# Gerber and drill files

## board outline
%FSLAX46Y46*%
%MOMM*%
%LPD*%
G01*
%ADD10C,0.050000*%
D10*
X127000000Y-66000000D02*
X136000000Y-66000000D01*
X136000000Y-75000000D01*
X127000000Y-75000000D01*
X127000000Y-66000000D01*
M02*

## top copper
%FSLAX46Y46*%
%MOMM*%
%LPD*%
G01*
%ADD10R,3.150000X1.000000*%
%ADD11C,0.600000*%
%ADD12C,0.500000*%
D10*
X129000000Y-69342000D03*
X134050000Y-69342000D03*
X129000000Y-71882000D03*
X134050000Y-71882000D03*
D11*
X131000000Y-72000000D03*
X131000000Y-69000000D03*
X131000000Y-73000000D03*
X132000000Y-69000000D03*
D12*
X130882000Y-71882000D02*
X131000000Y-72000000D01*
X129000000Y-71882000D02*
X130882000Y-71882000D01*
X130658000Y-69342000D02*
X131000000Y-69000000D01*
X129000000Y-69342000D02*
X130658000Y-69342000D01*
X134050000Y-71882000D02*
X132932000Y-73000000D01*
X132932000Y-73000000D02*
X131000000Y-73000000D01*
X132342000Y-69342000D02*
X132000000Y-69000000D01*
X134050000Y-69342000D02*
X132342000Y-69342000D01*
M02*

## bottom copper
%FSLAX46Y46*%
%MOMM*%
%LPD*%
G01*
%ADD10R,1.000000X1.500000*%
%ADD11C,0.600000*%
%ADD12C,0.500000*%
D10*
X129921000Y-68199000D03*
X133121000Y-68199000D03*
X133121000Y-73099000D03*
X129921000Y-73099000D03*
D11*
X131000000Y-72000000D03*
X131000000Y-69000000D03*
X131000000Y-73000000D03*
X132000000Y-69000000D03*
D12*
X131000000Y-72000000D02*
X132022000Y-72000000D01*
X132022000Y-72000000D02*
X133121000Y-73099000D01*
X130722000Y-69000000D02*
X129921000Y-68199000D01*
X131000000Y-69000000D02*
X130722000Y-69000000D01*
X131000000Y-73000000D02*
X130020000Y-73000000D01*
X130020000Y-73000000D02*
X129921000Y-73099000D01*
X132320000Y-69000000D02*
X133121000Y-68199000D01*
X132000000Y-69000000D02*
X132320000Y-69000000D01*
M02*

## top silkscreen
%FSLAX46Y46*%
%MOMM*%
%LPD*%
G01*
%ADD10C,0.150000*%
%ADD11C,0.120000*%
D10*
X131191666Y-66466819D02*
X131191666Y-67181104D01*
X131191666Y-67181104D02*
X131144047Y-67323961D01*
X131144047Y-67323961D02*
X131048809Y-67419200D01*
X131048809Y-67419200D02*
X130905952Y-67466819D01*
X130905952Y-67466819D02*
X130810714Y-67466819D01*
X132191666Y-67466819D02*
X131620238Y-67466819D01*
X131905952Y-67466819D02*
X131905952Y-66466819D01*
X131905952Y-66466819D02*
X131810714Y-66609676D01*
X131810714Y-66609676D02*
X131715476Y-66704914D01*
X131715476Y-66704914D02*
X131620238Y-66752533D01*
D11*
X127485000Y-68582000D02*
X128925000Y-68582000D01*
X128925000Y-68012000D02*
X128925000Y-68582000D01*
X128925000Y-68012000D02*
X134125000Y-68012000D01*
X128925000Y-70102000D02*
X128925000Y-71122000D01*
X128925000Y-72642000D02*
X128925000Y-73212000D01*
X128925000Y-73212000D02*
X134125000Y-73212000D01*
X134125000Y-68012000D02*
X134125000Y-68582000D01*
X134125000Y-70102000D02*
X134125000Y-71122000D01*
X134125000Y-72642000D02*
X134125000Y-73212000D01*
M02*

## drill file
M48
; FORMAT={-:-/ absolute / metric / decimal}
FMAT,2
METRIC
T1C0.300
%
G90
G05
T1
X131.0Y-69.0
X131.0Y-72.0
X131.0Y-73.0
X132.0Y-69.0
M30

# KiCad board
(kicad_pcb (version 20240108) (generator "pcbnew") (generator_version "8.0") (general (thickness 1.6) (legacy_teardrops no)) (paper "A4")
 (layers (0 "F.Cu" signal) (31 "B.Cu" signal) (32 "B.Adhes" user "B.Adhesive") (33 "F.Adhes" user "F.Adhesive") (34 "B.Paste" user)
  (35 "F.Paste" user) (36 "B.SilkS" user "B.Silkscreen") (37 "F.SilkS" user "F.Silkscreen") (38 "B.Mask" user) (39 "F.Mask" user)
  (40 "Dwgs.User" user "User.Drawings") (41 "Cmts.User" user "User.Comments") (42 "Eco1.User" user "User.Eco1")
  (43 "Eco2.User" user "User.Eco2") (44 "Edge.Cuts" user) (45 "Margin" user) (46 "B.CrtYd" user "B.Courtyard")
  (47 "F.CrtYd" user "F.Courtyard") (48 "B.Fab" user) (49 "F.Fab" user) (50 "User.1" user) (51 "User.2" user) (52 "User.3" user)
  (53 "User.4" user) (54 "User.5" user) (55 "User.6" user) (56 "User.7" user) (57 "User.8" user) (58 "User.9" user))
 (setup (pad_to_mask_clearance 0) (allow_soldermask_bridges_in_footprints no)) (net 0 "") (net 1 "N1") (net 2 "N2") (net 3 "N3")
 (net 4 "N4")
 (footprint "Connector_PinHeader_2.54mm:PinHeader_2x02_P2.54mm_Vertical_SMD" (layer "F.Cu") (at 131.525 70.612)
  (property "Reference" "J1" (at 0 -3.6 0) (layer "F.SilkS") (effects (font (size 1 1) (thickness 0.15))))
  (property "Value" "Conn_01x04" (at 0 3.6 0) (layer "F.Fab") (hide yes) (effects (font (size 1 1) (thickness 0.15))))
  (fp_line (start -4.04 -2.03) (end -2.6 -2.03) (stroke (width 0.12) (type solid)) (layer "F.SilkS"))
  (fp_line (start -2.6 -2.6) (end -2.6 -2.03) (stroke (width 0.12) (type solid)) (layer "F.SilkS"))
  (fp_line (start -2.6 -2.6) (end 2.6 -2.6) (stroke (width 0.12) (type solid)) (layer "F.SilkS"))
  (fp_line (start -2.6 -0.51) (end -2.6 0.51) (stroke (width 0.12) (type solid)) (layer "F.SilkS"))
  (fp_line (start -2.6 2.03) (end -2.6 2.6) (stroke (width 0.12) (type solid)) (layer "F.SilkS"))
  (fp_line (start -2.6 2.6) (end 2.6 2.6) (stroke (width 0.12) (type solid)) (layer "F.SilkS"))
  (fp_line (start 2.6 -2.6) (end 2.6 -2.03) (stroke (width 0.12) (type solid)) (layer "F.SilkS"))
  (fp_line (start 2.6 -0.51) (end 2.6 0.51) (stroke (width 0.12) (type solid)) (layer "F.SilkS"))
  (fp_line (start 2.6 2.03) (end 2.6 2.6) (stroke (width 0.12) (type solid)) (layer "F.SilkS"))
  (pad "1" smd rect (at -2.525 -1.27) (size 3.15 1) (layers "F.Cu" "F.Paste" "F.Mask") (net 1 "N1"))
  (pad "2" smd rect (at 2.525 -1.27) (size 3.15 1) (layers "F.Cu" "F.Paste" "F.Mask") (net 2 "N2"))
  (pad "3" smd rect (at -2.525 1.27) (size 3.15 1) (layers "F.Cu" "F.Paste" "F.Mask") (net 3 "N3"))
  (pad "4" smd rect (at 2.525 1.27) (size 3.15 1) (layers "F.Cu" "F.Paste" "F.Mask") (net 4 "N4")))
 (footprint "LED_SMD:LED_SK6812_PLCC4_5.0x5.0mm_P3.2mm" (layer "B.Cu") (at 131.521 70.649 90)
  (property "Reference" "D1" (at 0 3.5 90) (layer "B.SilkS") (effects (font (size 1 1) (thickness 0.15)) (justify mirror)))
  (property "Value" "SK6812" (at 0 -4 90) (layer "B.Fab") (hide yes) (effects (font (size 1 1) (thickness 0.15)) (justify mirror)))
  (pad "1" smd rect (at 2.45 -1.6 90) (size 1.5 1) (layers "B.Cu" "B.Paste" "B.Mask") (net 1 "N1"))
  (pad "2" smd rect (at 2.45 1.6 90) (size 1.5 1) (layers "B.Cu" "B.Paste" "B.Mask") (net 2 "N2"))
  (pad "3" smd rect (at -2.45 1.6 90) (size 1.5 1) (layers "B.Cu" "B.Paste" "B.Mask") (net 3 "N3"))
  (pad "4" smd rect (at -2.45 -1.6 90) (size 1.5 1) (layers "B.Cu" "B.Paste" "B.Mask") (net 4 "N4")))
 (gr_rect (start 127 66) (end 136 75) (stroke (width 0.05) (type default)) (fill none) (layer "Edge.Cuts"))
 (segment (start 130.882 71.882) (end 131 72) (width 0.5) (layer "F.Cu") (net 3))
 (segment (start 129 71.882) (end 130.882 71.882) (width 0.5) (layer "F.Cu") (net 3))
 (via (at 131 72) (size 0.6) (drill 0.3) (layers "F.Cu" "B.Cu") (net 3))
 (segment (start 131 72) (end 132.022 72) (width 0.5) (layer "B.Cu") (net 3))
 (segment (start 132.022 72) (end 133.121 73.099) (width 0.5) (layer "B.Cu") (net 3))
 (segment (start 130.658 69.342) (end 131 69) (width 0.5) (layer "F.Cu") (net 1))
 (segment (start 129 69.342) (end 130.658 69.342) (width 0.5) (layer "F.Cu") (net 1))
 (via (at 131 69) (size 0.6) (drill 0.3) (layers "F.Cu" "B.Cu") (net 1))
 (segment (start 130.722 69) (end 129.921 68.199) (width 0.5) (layer "B.Cu") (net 1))
 (segment (start 131 69) (end 130.722 69) (width 0.5) (layer "B.Cu") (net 1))
 (segment (start 134.05 71.882) (end 132.932 73) (width 0.5) (layer "F.Cu") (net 4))
 (segment (start 132.932 73) (end 131 73) (width 0.5) (layer "F.Cu") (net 4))
 (via (at 131 73) (size 0.6) (drill 0.3) (layers "F.Cu" "B.Cu") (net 4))
 (segment (start 131 73) (end 130.02 73) (width 0.5) (layer "B.Cu") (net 4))
 (segment (start 130.02 73) (end 129.921 73.099) (width 0.5) (layer "B.Cu") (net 4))
 (segment (start 132.342 69.342) (end 132 69) (width 0.5) (layer "F.Cu") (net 2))
 (segment (start 134.05 69.342) (end 132.342 69.342) (width 0.5) (layer "F.Cu") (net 2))
 (via (at 132 69) (size 0.6) (drill 0.3) (layers "F.Cu" "B.Cu") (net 2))
 (segment (start 132.32 69) (end 133.121 68.199) (width 0.5) (layer "B.Cu") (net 2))
 (segment (start 132 69) (end 132.32 69) (width 0.5) (layer "B.Cu") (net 2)))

